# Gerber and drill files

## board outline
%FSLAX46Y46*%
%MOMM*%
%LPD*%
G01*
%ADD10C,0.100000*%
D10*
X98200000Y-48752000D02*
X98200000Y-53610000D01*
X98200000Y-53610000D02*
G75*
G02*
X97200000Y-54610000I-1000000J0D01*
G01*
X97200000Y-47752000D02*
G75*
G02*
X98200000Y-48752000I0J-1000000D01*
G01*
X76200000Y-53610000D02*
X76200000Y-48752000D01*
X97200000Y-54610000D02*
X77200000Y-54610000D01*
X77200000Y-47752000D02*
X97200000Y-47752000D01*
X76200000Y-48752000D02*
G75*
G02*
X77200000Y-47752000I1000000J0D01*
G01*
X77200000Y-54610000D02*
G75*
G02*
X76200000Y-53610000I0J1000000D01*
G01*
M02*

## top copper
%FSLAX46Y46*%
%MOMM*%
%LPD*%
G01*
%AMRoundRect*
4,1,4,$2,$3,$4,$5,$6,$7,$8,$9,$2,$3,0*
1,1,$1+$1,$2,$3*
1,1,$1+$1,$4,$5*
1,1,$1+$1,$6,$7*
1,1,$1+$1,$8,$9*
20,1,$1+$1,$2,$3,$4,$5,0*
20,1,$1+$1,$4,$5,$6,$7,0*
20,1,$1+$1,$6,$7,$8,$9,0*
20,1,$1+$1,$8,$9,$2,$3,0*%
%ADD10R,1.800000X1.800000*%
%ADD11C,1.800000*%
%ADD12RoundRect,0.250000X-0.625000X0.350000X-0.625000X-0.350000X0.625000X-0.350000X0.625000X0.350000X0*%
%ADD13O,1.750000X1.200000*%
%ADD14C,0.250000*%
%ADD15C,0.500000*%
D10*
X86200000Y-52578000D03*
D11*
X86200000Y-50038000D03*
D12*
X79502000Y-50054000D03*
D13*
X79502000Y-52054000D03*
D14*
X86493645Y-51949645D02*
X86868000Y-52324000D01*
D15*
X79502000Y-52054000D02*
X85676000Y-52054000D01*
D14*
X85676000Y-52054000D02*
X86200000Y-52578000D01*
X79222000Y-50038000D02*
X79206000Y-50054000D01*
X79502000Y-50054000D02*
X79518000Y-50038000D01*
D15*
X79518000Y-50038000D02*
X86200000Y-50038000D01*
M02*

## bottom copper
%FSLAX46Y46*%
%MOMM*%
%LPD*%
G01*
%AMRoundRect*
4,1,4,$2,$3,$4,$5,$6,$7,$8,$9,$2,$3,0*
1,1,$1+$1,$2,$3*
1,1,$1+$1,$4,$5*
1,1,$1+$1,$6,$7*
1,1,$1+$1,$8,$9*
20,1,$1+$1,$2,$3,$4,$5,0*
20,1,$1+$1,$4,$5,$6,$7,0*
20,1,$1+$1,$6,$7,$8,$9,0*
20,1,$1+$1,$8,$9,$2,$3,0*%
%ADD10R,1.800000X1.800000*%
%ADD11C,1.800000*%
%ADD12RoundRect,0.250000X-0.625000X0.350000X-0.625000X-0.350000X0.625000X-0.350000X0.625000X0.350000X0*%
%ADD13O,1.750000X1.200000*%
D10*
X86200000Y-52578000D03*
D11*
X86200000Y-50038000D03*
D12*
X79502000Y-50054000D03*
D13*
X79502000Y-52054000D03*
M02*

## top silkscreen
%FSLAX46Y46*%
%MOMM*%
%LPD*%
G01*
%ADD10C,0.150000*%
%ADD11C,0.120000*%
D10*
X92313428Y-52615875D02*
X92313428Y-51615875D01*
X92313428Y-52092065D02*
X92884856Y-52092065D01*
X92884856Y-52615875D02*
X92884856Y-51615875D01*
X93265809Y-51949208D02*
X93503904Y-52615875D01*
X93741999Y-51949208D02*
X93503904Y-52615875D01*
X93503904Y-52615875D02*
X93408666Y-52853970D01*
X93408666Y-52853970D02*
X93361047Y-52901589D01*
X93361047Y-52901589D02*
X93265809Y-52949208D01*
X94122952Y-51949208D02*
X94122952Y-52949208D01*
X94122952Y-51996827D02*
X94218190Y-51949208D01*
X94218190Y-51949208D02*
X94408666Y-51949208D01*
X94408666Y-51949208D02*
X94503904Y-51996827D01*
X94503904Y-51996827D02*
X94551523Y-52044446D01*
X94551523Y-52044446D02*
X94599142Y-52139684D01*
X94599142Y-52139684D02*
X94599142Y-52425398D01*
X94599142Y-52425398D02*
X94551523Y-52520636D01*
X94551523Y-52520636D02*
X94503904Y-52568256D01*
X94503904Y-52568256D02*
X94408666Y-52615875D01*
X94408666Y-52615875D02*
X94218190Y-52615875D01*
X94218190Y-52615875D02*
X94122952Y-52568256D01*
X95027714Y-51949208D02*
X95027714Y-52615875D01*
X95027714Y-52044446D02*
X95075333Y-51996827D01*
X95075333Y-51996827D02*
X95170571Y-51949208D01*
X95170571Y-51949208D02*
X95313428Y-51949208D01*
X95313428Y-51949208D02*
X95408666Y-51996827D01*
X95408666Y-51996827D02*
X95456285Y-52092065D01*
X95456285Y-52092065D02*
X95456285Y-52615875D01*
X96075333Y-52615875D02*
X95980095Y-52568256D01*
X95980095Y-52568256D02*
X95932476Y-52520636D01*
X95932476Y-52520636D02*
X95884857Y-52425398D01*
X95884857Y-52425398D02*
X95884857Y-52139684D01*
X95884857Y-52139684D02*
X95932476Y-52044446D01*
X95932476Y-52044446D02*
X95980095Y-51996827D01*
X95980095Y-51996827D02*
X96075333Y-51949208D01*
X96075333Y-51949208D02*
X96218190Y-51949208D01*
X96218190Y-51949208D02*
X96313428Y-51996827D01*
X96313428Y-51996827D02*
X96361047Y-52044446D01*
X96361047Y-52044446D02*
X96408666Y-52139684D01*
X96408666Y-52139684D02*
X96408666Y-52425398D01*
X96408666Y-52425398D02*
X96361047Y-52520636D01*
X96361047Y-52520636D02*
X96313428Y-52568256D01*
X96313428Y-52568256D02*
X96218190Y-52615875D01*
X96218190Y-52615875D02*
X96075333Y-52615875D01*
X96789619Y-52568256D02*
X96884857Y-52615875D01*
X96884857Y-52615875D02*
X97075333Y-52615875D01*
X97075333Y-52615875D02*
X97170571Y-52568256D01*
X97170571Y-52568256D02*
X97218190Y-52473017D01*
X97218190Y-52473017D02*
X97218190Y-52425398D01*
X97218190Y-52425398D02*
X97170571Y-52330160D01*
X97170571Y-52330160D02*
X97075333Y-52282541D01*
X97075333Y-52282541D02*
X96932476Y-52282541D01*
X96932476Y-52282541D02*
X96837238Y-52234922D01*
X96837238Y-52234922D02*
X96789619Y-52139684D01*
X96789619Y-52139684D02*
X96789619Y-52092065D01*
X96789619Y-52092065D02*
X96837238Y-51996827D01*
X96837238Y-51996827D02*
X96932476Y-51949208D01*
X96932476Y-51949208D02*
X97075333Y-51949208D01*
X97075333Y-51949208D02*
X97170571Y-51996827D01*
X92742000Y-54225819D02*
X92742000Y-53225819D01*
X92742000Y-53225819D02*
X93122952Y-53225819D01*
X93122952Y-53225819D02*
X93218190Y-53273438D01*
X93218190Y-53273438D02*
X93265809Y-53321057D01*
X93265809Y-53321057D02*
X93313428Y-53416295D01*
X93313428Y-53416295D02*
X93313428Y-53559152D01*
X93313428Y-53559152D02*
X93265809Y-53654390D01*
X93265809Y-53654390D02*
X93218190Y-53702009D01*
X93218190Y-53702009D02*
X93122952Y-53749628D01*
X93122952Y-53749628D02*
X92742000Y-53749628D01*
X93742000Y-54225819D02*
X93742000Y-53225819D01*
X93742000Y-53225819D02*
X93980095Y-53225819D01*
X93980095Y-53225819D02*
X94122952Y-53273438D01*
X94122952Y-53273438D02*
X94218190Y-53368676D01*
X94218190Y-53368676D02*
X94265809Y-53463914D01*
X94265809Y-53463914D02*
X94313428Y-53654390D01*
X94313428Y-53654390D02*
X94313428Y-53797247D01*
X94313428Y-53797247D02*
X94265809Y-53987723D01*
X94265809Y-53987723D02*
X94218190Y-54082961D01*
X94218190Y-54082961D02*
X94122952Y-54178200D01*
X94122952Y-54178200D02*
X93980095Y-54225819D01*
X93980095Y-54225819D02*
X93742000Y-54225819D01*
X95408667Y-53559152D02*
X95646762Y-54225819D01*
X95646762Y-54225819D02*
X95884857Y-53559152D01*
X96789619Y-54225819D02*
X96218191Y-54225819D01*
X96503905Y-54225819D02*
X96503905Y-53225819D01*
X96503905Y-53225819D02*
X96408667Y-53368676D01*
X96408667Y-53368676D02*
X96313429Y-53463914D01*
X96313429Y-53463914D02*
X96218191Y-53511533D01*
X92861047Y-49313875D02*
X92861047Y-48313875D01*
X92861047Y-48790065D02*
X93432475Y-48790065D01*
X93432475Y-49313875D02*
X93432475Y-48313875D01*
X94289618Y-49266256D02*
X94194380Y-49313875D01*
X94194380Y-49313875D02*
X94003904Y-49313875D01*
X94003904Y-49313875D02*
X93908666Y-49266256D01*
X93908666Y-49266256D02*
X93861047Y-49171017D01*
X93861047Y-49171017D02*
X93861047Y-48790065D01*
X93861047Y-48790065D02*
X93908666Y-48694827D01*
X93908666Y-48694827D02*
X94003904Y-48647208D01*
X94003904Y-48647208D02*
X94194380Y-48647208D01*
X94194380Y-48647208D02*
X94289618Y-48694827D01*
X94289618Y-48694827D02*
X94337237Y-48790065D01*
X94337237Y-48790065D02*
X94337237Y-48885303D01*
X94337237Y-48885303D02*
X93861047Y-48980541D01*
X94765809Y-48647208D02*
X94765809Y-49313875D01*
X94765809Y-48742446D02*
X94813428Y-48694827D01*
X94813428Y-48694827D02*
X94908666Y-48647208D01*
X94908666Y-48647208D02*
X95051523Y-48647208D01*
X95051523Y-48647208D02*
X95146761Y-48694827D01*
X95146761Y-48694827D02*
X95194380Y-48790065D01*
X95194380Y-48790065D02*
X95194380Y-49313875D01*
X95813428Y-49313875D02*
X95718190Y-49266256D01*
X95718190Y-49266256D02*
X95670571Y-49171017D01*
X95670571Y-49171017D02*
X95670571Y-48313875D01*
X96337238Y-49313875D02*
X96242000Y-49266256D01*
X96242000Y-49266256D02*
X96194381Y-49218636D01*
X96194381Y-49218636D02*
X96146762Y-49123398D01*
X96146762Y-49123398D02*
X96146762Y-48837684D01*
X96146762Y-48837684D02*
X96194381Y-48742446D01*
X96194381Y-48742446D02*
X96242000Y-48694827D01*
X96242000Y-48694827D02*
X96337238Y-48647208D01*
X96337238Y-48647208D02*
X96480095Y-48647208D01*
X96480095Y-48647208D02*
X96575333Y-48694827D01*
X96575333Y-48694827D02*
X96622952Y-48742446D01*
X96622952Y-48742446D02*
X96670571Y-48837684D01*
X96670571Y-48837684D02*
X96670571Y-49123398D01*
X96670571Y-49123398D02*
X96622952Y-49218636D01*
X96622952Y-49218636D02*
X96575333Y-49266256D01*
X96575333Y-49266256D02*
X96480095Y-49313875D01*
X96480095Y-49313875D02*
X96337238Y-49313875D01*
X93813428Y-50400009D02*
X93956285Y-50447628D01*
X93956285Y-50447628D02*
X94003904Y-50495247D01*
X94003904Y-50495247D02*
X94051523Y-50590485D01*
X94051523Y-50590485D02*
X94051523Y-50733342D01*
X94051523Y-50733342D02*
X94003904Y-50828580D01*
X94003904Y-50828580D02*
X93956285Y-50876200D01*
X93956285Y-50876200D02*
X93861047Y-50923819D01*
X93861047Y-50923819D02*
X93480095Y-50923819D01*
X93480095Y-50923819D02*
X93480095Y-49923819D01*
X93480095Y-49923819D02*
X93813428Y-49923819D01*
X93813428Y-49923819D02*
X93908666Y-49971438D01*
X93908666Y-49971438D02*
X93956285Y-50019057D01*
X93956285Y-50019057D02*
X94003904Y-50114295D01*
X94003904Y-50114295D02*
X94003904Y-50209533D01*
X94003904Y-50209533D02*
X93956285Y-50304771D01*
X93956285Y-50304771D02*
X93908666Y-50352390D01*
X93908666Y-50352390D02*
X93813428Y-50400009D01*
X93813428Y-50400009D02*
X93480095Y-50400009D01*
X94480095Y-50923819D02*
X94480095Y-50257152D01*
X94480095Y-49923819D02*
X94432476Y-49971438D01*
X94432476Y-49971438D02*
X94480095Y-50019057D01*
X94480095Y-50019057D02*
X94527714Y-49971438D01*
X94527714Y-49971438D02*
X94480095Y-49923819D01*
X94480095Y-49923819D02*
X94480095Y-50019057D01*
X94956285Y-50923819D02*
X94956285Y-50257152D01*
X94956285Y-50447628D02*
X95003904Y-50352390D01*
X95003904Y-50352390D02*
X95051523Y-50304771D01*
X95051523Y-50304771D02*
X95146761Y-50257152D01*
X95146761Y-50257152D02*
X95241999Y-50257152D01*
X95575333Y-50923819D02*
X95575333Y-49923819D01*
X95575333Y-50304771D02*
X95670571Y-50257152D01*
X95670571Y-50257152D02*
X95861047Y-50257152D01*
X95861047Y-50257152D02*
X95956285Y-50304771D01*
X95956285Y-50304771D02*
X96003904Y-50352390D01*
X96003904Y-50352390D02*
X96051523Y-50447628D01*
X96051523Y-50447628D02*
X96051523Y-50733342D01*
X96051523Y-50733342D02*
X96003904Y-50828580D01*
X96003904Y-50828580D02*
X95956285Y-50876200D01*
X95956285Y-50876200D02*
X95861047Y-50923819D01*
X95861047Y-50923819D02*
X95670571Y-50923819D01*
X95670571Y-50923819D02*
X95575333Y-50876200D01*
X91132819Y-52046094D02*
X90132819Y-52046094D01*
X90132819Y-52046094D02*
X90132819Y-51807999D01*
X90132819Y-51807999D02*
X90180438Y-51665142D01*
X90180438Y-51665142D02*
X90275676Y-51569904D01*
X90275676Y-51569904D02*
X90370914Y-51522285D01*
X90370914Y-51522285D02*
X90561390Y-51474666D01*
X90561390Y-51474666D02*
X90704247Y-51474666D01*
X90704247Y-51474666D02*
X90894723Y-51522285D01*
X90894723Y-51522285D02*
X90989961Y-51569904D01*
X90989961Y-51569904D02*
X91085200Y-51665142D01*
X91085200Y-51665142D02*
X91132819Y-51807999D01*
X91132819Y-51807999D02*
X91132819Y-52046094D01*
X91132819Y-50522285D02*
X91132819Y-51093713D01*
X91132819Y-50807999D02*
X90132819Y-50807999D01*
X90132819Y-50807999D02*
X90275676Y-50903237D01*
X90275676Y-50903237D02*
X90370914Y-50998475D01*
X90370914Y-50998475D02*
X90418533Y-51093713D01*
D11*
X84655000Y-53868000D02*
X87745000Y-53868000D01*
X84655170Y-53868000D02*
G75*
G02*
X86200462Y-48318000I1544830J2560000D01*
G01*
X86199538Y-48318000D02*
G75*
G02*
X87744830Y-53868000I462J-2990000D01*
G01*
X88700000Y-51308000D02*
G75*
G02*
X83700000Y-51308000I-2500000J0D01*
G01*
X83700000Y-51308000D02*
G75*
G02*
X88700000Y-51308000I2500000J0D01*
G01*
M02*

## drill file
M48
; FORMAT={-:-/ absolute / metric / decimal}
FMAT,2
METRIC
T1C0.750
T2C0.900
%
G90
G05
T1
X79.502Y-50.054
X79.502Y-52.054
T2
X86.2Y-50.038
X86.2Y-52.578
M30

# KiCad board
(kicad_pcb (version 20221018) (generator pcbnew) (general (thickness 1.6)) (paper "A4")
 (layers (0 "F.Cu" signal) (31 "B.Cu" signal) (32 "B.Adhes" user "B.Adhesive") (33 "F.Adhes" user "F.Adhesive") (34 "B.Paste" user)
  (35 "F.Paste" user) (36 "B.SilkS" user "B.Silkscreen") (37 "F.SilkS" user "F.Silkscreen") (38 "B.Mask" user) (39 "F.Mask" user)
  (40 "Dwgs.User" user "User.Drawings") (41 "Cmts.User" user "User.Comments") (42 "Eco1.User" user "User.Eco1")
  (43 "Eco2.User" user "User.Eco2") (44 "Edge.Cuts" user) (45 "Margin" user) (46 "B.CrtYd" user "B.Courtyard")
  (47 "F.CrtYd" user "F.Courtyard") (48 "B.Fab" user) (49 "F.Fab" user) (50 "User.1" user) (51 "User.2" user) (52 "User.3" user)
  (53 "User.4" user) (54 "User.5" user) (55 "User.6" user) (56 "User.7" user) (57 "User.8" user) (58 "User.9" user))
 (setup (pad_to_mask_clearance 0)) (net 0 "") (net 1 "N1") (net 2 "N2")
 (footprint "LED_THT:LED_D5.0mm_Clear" (layer "F.Cu") (at 86.2 52.578 90)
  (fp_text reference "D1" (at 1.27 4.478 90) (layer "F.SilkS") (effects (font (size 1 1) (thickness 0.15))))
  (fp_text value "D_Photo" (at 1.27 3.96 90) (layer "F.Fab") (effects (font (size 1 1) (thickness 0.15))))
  (fp_line (start -1.29 -1.545) (end -1.29 1.545) (stroke (width 0.12) (type solid)) (layer "F.SilkS"))
  (fp_arc (start -1.29 -1.54483) (mid 2.072002 -2.880433) (end 4.26 0.000462) (stroke (width 0.12) (type solid)) (layer "F.SilkS"))
  (fp_arc (start 4.26 -0.000462) (mid 2.072002 2.880433) (end -1.29 1.54483) (stroke (width 0.12) (type solid)) (layer "F.SilkS"))
  (fp_circle (center 1.27 0) (end 3.77 0) (stroke (width 0.12) (type solid)) (fill none) (layer "F.SilkS"))
  (pad "1" thru_hole rect (at 0 0 90) (size 1.8 1.8) (drill 0.9) (layers "*.Cu" "*.Mask") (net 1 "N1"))
  (pad "2" thru_hole circle (at 2.54 0 90) (size 1.8 1.8) (drill 0.9) (layers "*.Cu" "*.Mask") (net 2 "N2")))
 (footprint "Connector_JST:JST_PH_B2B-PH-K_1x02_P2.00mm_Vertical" (layer "B.Cu") (at 79.502 50.054 -90)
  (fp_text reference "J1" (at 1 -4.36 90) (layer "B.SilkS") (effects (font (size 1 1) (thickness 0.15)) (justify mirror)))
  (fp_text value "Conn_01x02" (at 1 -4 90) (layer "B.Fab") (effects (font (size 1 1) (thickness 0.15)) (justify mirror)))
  (pad "1" thru_hole roundrect (at 0 0 270) (size 1.2 1.75) (drill 0.75) (layers "*.Cu" "*.Mask") (roundrect_rratio 0.2083333333)
   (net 2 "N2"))
  (pad "2" thru_hole oval (at 2 0 270) (size 1.2 1.75) (drill 0.75) (layers "*.Cu" "*.Mask") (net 1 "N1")))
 (gr_line (start 98.2 48.752) (end 98.2 53.61) (stroke (width 0.1) (type default)) (layer "Edge.Cuts"))
 (gr_arc (start 98.2 53.61) (mid 97.907107 54.317107) (end 97.2 54.61) (stroke (width 0.1) (type default)) (layer "Edge.Cuts"))
 (gr_arc (start 97.2 47.752) (mid 97.907107 48.044893) (end 98.2 48.752) (stroke (width 0.1) (type default)) (layer "Edge.Cuts"))
 (gr_line (start 76.2 53.61) (end 76.2 48.752) (stroke (width 0.1) (type default)) (layer "Edge.Cuts"))
 (gr_line (start 97.2 54.61) (end 77.2 54.61) (stroke (width 0.1) (type default)) (layer "Edge.Cuts"))
 (gr_line (start 77.2 47.752) (end 97.2 47.752) (stroke (width 0.1) (type default)) (layer "Edge.Cuts"))
 (gr_arc (start 76.2 48.752) (mid 76.492893 48.044893) (end 77.2 47.752) (stroke (width 0.1) (type default)) (layer "Edge.Cuts"))
 (gr_arc (start 77.2 54.61) (mid 76.492893 54.317107) (end 76.2 53.61) (stroke (width 0.1) (type default)) (layer "Edge.Cuts"))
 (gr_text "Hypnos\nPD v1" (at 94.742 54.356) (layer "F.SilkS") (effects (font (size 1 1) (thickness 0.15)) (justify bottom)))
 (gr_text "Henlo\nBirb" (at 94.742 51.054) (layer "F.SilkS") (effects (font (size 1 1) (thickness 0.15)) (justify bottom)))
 (segment (start 86.493645 51.949645) (end 86.868 52.324) (width 0.25) (layer "F.Cu") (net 1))
 (segment (start 79.502 52.054) (end 85.676 52.054) (width 0.5) (layer "F.Cu") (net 1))
 (segment (start 85.676 52.054) (end 86.2 52.578) (width 0.25) (layer "F.Cu") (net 1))
 (segment (start 79.222 50.038) (end 79.206 50.054) (width 0.25) (layer "F.Cu") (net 2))
 (segment (start 79.502 50.054) (end 79.518 50.038) (width 0.25) (layer "F.Cu") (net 2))
 (segment (start 79.518 50.038) (end 86.2 50.038) (width 0.5) (layer "F.Cu") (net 2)))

